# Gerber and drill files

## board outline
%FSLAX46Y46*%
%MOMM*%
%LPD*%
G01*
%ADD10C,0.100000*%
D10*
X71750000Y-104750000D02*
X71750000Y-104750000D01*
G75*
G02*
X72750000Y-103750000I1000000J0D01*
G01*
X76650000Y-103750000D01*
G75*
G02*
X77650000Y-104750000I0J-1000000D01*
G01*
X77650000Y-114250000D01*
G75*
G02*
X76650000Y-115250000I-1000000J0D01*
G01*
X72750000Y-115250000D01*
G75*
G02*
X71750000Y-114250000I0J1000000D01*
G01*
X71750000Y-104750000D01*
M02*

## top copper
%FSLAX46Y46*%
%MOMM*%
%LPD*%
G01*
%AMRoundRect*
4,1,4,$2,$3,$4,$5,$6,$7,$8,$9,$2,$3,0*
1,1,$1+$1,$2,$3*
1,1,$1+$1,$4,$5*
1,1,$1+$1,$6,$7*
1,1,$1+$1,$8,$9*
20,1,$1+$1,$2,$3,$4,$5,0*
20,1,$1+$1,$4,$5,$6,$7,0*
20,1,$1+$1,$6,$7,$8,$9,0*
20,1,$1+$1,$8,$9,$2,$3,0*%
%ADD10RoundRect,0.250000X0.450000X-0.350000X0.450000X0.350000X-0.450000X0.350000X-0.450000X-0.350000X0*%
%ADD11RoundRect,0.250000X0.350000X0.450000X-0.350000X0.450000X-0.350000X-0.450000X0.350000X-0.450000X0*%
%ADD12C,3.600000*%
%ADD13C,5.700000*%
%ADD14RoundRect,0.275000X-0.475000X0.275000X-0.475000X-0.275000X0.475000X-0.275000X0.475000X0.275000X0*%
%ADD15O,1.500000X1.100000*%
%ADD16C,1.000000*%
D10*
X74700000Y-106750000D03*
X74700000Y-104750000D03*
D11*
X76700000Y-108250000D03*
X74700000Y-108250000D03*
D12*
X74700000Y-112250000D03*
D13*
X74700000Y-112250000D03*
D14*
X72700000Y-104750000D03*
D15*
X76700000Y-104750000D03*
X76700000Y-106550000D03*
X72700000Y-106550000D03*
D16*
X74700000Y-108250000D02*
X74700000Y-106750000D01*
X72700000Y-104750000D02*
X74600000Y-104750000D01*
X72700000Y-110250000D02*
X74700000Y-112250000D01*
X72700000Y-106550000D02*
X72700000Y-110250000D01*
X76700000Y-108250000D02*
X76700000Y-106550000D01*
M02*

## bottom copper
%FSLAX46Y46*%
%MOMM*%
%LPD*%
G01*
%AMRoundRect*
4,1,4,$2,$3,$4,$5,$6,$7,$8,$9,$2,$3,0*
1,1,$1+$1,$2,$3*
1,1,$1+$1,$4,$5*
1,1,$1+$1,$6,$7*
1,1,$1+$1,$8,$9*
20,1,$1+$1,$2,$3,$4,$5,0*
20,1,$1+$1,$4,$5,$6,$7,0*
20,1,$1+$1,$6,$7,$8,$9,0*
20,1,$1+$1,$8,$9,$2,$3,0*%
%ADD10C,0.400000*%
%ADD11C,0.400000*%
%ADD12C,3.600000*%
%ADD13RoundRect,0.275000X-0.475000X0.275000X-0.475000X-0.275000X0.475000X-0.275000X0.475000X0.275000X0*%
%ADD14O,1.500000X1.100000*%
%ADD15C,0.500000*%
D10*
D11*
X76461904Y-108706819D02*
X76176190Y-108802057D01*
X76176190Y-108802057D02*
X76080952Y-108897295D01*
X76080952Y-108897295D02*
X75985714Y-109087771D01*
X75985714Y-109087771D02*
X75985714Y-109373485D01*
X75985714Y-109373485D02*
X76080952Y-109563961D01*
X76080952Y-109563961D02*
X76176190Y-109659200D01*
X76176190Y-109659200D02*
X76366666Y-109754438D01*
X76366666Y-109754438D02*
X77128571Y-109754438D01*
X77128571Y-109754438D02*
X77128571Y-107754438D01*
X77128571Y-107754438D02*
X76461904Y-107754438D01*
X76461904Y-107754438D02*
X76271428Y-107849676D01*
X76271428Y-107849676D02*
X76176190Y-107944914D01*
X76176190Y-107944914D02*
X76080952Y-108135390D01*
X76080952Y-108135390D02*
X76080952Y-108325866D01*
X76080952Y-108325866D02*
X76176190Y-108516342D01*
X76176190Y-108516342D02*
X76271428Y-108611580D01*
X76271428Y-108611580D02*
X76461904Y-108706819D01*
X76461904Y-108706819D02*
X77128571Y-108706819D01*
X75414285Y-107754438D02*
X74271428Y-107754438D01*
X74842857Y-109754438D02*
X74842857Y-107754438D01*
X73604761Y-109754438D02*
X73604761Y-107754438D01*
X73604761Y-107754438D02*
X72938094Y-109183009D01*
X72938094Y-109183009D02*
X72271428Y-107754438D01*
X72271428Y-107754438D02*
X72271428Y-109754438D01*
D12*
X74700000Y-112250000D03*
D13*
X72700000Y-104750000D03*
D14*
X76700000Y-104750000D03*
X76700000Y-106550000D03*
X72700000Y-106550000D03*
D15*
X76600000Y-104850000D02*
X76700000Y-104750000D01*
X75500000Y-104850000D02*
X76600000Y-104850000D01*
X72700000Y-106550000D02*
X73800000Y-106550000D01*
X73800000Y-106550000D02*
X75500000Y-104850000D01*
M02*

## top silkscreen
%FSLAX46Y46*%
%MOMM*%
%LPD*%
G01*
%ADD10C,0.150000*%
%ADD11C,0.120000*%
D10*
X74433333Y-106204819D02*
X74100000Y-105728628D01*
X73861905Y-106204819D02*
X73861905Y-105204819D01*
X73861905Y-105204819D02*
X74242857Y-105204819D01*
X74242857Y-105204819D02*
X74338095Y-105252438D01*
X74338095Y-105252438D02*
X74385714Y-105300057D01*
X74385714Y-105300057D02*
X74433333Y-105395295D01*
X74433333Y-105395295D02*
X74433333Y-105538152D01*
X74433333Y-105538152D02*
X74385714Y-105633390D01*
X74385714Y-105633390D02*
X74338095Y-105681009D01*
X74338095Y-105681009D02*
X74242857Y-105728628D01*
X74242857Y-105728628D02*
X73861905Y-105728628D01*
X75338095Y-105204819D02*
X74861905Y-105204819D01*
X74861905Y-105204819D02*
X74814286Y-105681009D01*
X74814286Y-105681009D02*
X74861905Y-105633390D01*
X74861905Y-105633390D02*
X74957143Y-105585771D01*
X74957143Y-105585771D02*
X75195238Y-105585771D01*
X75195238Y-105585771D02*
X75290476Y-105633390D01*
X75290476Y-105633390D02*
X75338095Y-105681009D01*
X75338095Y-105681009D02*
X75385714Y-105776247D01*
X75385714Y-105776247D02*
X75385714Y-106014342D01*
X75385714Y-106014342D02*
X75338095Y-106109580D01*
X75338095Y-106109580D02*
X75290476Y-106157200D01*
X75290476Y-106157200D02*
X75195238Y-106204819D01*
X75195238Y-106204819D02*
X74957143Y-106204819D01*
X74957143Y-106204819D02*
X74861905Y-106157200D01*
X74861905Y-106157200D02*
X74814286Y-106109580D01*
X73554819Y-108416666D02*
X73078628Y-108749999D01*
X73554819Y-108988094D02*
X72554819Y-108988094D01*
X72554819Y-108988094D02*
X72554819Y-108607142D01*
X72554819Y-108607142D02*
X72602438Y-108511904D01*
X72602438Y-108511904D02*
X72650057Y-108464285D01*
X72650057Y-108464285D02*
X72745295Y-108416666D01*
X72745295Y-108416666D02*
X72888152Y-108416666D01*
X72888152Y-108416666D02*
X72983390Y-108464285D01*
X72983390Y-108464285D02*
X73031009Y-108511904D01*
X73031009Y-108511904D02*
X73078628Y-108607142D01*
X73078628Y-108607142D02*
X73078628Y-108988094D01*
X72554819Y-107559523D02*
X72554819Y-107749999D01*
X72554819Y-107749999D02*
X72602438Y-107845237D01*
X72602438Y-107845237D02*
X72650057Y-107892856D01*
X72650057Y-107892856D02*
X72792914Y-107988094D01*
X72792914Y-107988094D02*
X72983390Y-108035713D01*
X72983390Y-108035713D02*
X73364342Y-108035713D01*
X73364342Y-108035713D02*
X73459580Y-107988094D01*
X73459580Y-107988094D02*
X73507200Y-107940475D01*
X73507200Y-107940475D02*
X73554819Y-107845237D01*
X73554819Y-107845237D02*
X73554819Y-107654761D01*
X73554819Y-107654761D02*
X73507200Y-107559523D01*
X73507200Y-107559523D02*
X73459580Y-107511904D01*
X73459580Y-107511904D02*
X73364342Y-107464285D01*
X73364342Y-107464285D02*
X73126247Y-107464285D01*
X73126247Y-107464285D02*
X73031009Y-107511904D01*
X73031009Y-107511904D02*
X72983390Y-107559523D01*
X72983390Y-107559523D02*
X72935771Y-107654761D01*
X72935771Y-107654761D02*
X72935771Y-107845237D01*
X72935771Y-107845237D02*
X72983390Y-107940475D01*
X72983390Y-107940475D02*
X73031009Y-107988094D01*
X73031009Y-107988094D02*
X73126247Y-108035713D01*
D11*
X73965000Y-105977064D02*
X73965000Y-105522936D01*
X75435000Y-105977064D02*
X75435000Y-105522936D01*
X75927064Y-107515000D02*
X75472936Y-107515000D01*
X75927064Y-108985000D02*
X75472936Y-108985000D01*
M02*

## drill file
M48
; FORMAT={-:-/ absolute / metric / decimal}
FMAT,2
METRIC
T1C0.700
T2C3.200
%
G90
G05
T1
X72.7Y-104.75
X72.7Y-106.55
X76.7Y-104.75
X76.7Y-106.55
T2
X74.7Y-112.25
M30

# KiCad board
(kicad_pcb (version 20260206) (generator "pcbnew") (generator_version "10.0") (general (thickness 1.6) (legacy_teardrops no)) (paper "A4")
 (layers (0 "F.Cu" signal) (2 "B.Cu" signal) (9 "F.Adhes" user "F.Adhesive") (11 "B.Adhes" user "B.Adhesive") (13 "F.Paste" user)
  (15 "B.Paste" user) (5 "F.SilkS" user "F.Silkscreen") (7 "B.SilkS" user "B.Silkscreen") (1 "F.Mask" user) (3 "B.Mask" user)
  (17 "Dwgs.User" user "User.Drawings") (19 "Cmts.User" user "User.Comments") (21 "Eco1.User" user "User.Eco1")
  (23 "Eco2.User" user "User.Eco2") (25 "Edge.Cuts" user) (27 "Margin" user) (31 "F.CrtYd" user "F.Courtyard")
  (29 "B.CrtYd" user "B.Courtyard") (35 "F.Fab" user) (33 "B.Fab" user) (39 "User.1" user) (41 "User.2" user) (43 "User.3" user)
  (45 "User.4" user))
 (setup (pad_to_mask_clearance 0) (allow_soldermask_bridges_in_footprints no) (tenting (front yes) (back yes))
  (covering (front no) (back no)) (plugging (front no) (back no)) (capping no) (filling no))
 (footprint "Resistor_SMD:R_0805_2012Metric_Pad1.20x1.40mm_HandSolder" (layer "F.Cu") (at 74.7 105.75 90)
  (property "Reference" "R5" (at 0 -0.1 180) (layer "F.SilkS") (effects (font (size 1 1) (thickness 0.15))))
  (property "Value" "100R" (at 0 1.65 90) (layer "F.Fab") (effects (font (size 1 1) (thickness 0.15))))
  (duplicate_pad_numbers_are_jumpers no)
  (fp_line (start -0.227064 -0.735) (end 0.227064 -0.735) (stroke (width 0.12) (type solid)) (layer "F.SilkS"))
  (fp_line (start -0.227064 0.735) (end 0.227064 0.735) (stroke (width 0.12) (type solid)) (layer "F.SilkS"))
  (pad "1" smd roundrect (at -1 0 90) (size 1.2 1.4) (layers "F.Cu" "F.Mask" "F.Paste") (roundrect_rratio 0.208333) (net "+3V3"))
  (pad "2" smd roundrect (at 1 0 90) (size 1.2 1.4) (layers "F.Cu" "F.Mask" "F.Paste") (roundrect_rratio 0.208333) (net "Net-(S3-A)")))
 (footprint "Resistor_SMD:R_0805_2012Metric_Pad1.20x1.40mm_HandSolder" (layer "F.Cu") (at 75.7 108.25 180)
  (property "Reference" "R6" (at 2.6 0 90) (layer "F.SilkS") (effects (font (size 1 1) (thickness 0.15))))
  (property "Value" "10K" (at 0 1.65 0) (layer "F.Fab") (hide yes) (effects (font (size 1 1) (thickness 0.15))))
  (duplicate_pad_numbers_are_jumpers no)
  (fp_line (start -0.227064 0.735) (end 0.227064 0.735) (stroke (width 0.12) (type solid)) (layer "F.SilkS"))
  (fp_line (start -0.227064 -0.735) (end 0.227064 -0.735) (stroke (width 0.12) (type solid)) (layer "F.SilkS"))
  (pad "1" smd roundrect (at -1 0 180) (size 1.2 1.4) (layers "F.Cu" "F.Mask" "F.Paste") (roundrect_rratio 0.208333) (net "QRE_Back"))
  (pad "2" smd roundrect (at 1 0 180) (size 1.2 1.4) (layers "F.Cu" "F.Mask" "F.Paste") (roundrect_rratio 0.208333) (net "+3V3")))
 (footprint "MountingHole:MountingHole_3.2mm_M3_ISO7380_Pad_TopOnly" (layer "F.Cu") (at 74.7 112.25)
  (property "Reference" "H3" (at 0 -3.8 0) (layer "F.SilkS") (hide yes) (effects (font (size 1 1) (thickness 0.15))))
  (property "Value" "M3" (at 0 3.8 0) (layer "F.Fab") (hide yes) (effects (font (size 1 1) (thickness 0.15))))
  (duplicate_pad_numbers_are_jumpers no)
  (pad "1" thru_hole circle (at 0 0) (size 3.6 3.6) (drill 3.2) (layers "*.Cu" "*.Mask") (remove_unused_layers no) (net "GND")
   (zone_connect 2))
  (pad "1" connect circle (at 0 0) (size 5.7 5.7) (layers "F.Cu" "F.Mask") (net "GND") (zone_connect 2)))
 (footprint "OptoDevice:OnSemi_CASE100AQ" (layer "B.Cu") (at 72.7 104.75 -90)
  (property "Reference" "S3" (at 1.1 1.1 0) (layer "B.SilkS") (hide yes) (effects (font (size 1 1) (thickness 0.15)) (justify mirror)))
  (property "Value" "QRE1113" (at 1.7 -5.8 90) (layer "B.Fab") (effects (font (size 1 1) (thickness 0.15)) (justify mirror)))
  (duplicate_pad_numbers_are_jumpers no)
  (pad "1" thru_hole roundrect (at 0 0 270) (size 1.1 1.5) (drill 0.7) (layers "*.Cu" "*.Mask") (remove_unused_layers no)
   (roundrect_rratio 0.25) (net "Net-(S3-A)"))
  (pad "2" thru_hole oval (at 0 -4 270) (size 1.1 1.5) (drill 0.7) (layers "*.Cu" "*.Mask") (remove_unused_layers no) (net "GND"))
  (pad "3" thru_hole oval (at 1.8 -4 270) (size 1.1 1.5) (drill 0.7) (layers "*.Cu" "*.Mask") (remove_unused_layers no) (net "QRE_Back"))
  (pad "4" thru_hole oval (at 1.8 0 270) (size 1.1 1.5) (drill 0.7) (layers "*.Cu" "*.Mask") (remove_unused_layers no) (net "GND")))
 (gr_rect (start 71.75 103.75) (end 77.65 115.25) (radius 1) (stroke (width 0.1) (type solid)) (fill no) (layer "Edge.Cuts"))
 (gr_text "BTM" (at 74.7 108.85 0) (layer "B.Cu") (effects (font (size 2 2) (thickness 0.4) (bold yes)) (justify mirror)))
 (segment (start 74.7 108.25) (end 74.7 106.75) (width 1) (layer "F.Cu") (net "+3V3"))
 (segment (start 72.7 104.75) (end 74.6 104.75) (width 1) (layer "F.Cu") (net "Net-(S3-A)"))
 (segment (start 72.7 110.25) (end 74.7 112.25) (width 1) (layer "F.Cu") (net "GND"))
 (segment (start 72.7 106.55) (end 72.7 110.25) (width 1) (layer "F.Cu") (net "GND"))
 (segment (start 76.6 104.85) (end 76.7 104.75) (width 0.5) (layer "B.Cu") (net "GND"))
 (segment (start 75.5 104.85) (end 76.6 104.85) (width 0.5) (layer "B.Cu") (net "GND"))
 (segment (start 72.7 106.55) (end 73.8 106.55) (width 0.5) (layer "B.Cu") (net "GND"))
 (segment (start 73.8 106.55) (end 75.5 104.85) (width 0.5) (layer "B.Cu") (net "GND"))
 (segment (start 76.7 108.25) (end 76.7 106.55) (width 1) (layer "F.Cu") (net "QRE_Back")))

